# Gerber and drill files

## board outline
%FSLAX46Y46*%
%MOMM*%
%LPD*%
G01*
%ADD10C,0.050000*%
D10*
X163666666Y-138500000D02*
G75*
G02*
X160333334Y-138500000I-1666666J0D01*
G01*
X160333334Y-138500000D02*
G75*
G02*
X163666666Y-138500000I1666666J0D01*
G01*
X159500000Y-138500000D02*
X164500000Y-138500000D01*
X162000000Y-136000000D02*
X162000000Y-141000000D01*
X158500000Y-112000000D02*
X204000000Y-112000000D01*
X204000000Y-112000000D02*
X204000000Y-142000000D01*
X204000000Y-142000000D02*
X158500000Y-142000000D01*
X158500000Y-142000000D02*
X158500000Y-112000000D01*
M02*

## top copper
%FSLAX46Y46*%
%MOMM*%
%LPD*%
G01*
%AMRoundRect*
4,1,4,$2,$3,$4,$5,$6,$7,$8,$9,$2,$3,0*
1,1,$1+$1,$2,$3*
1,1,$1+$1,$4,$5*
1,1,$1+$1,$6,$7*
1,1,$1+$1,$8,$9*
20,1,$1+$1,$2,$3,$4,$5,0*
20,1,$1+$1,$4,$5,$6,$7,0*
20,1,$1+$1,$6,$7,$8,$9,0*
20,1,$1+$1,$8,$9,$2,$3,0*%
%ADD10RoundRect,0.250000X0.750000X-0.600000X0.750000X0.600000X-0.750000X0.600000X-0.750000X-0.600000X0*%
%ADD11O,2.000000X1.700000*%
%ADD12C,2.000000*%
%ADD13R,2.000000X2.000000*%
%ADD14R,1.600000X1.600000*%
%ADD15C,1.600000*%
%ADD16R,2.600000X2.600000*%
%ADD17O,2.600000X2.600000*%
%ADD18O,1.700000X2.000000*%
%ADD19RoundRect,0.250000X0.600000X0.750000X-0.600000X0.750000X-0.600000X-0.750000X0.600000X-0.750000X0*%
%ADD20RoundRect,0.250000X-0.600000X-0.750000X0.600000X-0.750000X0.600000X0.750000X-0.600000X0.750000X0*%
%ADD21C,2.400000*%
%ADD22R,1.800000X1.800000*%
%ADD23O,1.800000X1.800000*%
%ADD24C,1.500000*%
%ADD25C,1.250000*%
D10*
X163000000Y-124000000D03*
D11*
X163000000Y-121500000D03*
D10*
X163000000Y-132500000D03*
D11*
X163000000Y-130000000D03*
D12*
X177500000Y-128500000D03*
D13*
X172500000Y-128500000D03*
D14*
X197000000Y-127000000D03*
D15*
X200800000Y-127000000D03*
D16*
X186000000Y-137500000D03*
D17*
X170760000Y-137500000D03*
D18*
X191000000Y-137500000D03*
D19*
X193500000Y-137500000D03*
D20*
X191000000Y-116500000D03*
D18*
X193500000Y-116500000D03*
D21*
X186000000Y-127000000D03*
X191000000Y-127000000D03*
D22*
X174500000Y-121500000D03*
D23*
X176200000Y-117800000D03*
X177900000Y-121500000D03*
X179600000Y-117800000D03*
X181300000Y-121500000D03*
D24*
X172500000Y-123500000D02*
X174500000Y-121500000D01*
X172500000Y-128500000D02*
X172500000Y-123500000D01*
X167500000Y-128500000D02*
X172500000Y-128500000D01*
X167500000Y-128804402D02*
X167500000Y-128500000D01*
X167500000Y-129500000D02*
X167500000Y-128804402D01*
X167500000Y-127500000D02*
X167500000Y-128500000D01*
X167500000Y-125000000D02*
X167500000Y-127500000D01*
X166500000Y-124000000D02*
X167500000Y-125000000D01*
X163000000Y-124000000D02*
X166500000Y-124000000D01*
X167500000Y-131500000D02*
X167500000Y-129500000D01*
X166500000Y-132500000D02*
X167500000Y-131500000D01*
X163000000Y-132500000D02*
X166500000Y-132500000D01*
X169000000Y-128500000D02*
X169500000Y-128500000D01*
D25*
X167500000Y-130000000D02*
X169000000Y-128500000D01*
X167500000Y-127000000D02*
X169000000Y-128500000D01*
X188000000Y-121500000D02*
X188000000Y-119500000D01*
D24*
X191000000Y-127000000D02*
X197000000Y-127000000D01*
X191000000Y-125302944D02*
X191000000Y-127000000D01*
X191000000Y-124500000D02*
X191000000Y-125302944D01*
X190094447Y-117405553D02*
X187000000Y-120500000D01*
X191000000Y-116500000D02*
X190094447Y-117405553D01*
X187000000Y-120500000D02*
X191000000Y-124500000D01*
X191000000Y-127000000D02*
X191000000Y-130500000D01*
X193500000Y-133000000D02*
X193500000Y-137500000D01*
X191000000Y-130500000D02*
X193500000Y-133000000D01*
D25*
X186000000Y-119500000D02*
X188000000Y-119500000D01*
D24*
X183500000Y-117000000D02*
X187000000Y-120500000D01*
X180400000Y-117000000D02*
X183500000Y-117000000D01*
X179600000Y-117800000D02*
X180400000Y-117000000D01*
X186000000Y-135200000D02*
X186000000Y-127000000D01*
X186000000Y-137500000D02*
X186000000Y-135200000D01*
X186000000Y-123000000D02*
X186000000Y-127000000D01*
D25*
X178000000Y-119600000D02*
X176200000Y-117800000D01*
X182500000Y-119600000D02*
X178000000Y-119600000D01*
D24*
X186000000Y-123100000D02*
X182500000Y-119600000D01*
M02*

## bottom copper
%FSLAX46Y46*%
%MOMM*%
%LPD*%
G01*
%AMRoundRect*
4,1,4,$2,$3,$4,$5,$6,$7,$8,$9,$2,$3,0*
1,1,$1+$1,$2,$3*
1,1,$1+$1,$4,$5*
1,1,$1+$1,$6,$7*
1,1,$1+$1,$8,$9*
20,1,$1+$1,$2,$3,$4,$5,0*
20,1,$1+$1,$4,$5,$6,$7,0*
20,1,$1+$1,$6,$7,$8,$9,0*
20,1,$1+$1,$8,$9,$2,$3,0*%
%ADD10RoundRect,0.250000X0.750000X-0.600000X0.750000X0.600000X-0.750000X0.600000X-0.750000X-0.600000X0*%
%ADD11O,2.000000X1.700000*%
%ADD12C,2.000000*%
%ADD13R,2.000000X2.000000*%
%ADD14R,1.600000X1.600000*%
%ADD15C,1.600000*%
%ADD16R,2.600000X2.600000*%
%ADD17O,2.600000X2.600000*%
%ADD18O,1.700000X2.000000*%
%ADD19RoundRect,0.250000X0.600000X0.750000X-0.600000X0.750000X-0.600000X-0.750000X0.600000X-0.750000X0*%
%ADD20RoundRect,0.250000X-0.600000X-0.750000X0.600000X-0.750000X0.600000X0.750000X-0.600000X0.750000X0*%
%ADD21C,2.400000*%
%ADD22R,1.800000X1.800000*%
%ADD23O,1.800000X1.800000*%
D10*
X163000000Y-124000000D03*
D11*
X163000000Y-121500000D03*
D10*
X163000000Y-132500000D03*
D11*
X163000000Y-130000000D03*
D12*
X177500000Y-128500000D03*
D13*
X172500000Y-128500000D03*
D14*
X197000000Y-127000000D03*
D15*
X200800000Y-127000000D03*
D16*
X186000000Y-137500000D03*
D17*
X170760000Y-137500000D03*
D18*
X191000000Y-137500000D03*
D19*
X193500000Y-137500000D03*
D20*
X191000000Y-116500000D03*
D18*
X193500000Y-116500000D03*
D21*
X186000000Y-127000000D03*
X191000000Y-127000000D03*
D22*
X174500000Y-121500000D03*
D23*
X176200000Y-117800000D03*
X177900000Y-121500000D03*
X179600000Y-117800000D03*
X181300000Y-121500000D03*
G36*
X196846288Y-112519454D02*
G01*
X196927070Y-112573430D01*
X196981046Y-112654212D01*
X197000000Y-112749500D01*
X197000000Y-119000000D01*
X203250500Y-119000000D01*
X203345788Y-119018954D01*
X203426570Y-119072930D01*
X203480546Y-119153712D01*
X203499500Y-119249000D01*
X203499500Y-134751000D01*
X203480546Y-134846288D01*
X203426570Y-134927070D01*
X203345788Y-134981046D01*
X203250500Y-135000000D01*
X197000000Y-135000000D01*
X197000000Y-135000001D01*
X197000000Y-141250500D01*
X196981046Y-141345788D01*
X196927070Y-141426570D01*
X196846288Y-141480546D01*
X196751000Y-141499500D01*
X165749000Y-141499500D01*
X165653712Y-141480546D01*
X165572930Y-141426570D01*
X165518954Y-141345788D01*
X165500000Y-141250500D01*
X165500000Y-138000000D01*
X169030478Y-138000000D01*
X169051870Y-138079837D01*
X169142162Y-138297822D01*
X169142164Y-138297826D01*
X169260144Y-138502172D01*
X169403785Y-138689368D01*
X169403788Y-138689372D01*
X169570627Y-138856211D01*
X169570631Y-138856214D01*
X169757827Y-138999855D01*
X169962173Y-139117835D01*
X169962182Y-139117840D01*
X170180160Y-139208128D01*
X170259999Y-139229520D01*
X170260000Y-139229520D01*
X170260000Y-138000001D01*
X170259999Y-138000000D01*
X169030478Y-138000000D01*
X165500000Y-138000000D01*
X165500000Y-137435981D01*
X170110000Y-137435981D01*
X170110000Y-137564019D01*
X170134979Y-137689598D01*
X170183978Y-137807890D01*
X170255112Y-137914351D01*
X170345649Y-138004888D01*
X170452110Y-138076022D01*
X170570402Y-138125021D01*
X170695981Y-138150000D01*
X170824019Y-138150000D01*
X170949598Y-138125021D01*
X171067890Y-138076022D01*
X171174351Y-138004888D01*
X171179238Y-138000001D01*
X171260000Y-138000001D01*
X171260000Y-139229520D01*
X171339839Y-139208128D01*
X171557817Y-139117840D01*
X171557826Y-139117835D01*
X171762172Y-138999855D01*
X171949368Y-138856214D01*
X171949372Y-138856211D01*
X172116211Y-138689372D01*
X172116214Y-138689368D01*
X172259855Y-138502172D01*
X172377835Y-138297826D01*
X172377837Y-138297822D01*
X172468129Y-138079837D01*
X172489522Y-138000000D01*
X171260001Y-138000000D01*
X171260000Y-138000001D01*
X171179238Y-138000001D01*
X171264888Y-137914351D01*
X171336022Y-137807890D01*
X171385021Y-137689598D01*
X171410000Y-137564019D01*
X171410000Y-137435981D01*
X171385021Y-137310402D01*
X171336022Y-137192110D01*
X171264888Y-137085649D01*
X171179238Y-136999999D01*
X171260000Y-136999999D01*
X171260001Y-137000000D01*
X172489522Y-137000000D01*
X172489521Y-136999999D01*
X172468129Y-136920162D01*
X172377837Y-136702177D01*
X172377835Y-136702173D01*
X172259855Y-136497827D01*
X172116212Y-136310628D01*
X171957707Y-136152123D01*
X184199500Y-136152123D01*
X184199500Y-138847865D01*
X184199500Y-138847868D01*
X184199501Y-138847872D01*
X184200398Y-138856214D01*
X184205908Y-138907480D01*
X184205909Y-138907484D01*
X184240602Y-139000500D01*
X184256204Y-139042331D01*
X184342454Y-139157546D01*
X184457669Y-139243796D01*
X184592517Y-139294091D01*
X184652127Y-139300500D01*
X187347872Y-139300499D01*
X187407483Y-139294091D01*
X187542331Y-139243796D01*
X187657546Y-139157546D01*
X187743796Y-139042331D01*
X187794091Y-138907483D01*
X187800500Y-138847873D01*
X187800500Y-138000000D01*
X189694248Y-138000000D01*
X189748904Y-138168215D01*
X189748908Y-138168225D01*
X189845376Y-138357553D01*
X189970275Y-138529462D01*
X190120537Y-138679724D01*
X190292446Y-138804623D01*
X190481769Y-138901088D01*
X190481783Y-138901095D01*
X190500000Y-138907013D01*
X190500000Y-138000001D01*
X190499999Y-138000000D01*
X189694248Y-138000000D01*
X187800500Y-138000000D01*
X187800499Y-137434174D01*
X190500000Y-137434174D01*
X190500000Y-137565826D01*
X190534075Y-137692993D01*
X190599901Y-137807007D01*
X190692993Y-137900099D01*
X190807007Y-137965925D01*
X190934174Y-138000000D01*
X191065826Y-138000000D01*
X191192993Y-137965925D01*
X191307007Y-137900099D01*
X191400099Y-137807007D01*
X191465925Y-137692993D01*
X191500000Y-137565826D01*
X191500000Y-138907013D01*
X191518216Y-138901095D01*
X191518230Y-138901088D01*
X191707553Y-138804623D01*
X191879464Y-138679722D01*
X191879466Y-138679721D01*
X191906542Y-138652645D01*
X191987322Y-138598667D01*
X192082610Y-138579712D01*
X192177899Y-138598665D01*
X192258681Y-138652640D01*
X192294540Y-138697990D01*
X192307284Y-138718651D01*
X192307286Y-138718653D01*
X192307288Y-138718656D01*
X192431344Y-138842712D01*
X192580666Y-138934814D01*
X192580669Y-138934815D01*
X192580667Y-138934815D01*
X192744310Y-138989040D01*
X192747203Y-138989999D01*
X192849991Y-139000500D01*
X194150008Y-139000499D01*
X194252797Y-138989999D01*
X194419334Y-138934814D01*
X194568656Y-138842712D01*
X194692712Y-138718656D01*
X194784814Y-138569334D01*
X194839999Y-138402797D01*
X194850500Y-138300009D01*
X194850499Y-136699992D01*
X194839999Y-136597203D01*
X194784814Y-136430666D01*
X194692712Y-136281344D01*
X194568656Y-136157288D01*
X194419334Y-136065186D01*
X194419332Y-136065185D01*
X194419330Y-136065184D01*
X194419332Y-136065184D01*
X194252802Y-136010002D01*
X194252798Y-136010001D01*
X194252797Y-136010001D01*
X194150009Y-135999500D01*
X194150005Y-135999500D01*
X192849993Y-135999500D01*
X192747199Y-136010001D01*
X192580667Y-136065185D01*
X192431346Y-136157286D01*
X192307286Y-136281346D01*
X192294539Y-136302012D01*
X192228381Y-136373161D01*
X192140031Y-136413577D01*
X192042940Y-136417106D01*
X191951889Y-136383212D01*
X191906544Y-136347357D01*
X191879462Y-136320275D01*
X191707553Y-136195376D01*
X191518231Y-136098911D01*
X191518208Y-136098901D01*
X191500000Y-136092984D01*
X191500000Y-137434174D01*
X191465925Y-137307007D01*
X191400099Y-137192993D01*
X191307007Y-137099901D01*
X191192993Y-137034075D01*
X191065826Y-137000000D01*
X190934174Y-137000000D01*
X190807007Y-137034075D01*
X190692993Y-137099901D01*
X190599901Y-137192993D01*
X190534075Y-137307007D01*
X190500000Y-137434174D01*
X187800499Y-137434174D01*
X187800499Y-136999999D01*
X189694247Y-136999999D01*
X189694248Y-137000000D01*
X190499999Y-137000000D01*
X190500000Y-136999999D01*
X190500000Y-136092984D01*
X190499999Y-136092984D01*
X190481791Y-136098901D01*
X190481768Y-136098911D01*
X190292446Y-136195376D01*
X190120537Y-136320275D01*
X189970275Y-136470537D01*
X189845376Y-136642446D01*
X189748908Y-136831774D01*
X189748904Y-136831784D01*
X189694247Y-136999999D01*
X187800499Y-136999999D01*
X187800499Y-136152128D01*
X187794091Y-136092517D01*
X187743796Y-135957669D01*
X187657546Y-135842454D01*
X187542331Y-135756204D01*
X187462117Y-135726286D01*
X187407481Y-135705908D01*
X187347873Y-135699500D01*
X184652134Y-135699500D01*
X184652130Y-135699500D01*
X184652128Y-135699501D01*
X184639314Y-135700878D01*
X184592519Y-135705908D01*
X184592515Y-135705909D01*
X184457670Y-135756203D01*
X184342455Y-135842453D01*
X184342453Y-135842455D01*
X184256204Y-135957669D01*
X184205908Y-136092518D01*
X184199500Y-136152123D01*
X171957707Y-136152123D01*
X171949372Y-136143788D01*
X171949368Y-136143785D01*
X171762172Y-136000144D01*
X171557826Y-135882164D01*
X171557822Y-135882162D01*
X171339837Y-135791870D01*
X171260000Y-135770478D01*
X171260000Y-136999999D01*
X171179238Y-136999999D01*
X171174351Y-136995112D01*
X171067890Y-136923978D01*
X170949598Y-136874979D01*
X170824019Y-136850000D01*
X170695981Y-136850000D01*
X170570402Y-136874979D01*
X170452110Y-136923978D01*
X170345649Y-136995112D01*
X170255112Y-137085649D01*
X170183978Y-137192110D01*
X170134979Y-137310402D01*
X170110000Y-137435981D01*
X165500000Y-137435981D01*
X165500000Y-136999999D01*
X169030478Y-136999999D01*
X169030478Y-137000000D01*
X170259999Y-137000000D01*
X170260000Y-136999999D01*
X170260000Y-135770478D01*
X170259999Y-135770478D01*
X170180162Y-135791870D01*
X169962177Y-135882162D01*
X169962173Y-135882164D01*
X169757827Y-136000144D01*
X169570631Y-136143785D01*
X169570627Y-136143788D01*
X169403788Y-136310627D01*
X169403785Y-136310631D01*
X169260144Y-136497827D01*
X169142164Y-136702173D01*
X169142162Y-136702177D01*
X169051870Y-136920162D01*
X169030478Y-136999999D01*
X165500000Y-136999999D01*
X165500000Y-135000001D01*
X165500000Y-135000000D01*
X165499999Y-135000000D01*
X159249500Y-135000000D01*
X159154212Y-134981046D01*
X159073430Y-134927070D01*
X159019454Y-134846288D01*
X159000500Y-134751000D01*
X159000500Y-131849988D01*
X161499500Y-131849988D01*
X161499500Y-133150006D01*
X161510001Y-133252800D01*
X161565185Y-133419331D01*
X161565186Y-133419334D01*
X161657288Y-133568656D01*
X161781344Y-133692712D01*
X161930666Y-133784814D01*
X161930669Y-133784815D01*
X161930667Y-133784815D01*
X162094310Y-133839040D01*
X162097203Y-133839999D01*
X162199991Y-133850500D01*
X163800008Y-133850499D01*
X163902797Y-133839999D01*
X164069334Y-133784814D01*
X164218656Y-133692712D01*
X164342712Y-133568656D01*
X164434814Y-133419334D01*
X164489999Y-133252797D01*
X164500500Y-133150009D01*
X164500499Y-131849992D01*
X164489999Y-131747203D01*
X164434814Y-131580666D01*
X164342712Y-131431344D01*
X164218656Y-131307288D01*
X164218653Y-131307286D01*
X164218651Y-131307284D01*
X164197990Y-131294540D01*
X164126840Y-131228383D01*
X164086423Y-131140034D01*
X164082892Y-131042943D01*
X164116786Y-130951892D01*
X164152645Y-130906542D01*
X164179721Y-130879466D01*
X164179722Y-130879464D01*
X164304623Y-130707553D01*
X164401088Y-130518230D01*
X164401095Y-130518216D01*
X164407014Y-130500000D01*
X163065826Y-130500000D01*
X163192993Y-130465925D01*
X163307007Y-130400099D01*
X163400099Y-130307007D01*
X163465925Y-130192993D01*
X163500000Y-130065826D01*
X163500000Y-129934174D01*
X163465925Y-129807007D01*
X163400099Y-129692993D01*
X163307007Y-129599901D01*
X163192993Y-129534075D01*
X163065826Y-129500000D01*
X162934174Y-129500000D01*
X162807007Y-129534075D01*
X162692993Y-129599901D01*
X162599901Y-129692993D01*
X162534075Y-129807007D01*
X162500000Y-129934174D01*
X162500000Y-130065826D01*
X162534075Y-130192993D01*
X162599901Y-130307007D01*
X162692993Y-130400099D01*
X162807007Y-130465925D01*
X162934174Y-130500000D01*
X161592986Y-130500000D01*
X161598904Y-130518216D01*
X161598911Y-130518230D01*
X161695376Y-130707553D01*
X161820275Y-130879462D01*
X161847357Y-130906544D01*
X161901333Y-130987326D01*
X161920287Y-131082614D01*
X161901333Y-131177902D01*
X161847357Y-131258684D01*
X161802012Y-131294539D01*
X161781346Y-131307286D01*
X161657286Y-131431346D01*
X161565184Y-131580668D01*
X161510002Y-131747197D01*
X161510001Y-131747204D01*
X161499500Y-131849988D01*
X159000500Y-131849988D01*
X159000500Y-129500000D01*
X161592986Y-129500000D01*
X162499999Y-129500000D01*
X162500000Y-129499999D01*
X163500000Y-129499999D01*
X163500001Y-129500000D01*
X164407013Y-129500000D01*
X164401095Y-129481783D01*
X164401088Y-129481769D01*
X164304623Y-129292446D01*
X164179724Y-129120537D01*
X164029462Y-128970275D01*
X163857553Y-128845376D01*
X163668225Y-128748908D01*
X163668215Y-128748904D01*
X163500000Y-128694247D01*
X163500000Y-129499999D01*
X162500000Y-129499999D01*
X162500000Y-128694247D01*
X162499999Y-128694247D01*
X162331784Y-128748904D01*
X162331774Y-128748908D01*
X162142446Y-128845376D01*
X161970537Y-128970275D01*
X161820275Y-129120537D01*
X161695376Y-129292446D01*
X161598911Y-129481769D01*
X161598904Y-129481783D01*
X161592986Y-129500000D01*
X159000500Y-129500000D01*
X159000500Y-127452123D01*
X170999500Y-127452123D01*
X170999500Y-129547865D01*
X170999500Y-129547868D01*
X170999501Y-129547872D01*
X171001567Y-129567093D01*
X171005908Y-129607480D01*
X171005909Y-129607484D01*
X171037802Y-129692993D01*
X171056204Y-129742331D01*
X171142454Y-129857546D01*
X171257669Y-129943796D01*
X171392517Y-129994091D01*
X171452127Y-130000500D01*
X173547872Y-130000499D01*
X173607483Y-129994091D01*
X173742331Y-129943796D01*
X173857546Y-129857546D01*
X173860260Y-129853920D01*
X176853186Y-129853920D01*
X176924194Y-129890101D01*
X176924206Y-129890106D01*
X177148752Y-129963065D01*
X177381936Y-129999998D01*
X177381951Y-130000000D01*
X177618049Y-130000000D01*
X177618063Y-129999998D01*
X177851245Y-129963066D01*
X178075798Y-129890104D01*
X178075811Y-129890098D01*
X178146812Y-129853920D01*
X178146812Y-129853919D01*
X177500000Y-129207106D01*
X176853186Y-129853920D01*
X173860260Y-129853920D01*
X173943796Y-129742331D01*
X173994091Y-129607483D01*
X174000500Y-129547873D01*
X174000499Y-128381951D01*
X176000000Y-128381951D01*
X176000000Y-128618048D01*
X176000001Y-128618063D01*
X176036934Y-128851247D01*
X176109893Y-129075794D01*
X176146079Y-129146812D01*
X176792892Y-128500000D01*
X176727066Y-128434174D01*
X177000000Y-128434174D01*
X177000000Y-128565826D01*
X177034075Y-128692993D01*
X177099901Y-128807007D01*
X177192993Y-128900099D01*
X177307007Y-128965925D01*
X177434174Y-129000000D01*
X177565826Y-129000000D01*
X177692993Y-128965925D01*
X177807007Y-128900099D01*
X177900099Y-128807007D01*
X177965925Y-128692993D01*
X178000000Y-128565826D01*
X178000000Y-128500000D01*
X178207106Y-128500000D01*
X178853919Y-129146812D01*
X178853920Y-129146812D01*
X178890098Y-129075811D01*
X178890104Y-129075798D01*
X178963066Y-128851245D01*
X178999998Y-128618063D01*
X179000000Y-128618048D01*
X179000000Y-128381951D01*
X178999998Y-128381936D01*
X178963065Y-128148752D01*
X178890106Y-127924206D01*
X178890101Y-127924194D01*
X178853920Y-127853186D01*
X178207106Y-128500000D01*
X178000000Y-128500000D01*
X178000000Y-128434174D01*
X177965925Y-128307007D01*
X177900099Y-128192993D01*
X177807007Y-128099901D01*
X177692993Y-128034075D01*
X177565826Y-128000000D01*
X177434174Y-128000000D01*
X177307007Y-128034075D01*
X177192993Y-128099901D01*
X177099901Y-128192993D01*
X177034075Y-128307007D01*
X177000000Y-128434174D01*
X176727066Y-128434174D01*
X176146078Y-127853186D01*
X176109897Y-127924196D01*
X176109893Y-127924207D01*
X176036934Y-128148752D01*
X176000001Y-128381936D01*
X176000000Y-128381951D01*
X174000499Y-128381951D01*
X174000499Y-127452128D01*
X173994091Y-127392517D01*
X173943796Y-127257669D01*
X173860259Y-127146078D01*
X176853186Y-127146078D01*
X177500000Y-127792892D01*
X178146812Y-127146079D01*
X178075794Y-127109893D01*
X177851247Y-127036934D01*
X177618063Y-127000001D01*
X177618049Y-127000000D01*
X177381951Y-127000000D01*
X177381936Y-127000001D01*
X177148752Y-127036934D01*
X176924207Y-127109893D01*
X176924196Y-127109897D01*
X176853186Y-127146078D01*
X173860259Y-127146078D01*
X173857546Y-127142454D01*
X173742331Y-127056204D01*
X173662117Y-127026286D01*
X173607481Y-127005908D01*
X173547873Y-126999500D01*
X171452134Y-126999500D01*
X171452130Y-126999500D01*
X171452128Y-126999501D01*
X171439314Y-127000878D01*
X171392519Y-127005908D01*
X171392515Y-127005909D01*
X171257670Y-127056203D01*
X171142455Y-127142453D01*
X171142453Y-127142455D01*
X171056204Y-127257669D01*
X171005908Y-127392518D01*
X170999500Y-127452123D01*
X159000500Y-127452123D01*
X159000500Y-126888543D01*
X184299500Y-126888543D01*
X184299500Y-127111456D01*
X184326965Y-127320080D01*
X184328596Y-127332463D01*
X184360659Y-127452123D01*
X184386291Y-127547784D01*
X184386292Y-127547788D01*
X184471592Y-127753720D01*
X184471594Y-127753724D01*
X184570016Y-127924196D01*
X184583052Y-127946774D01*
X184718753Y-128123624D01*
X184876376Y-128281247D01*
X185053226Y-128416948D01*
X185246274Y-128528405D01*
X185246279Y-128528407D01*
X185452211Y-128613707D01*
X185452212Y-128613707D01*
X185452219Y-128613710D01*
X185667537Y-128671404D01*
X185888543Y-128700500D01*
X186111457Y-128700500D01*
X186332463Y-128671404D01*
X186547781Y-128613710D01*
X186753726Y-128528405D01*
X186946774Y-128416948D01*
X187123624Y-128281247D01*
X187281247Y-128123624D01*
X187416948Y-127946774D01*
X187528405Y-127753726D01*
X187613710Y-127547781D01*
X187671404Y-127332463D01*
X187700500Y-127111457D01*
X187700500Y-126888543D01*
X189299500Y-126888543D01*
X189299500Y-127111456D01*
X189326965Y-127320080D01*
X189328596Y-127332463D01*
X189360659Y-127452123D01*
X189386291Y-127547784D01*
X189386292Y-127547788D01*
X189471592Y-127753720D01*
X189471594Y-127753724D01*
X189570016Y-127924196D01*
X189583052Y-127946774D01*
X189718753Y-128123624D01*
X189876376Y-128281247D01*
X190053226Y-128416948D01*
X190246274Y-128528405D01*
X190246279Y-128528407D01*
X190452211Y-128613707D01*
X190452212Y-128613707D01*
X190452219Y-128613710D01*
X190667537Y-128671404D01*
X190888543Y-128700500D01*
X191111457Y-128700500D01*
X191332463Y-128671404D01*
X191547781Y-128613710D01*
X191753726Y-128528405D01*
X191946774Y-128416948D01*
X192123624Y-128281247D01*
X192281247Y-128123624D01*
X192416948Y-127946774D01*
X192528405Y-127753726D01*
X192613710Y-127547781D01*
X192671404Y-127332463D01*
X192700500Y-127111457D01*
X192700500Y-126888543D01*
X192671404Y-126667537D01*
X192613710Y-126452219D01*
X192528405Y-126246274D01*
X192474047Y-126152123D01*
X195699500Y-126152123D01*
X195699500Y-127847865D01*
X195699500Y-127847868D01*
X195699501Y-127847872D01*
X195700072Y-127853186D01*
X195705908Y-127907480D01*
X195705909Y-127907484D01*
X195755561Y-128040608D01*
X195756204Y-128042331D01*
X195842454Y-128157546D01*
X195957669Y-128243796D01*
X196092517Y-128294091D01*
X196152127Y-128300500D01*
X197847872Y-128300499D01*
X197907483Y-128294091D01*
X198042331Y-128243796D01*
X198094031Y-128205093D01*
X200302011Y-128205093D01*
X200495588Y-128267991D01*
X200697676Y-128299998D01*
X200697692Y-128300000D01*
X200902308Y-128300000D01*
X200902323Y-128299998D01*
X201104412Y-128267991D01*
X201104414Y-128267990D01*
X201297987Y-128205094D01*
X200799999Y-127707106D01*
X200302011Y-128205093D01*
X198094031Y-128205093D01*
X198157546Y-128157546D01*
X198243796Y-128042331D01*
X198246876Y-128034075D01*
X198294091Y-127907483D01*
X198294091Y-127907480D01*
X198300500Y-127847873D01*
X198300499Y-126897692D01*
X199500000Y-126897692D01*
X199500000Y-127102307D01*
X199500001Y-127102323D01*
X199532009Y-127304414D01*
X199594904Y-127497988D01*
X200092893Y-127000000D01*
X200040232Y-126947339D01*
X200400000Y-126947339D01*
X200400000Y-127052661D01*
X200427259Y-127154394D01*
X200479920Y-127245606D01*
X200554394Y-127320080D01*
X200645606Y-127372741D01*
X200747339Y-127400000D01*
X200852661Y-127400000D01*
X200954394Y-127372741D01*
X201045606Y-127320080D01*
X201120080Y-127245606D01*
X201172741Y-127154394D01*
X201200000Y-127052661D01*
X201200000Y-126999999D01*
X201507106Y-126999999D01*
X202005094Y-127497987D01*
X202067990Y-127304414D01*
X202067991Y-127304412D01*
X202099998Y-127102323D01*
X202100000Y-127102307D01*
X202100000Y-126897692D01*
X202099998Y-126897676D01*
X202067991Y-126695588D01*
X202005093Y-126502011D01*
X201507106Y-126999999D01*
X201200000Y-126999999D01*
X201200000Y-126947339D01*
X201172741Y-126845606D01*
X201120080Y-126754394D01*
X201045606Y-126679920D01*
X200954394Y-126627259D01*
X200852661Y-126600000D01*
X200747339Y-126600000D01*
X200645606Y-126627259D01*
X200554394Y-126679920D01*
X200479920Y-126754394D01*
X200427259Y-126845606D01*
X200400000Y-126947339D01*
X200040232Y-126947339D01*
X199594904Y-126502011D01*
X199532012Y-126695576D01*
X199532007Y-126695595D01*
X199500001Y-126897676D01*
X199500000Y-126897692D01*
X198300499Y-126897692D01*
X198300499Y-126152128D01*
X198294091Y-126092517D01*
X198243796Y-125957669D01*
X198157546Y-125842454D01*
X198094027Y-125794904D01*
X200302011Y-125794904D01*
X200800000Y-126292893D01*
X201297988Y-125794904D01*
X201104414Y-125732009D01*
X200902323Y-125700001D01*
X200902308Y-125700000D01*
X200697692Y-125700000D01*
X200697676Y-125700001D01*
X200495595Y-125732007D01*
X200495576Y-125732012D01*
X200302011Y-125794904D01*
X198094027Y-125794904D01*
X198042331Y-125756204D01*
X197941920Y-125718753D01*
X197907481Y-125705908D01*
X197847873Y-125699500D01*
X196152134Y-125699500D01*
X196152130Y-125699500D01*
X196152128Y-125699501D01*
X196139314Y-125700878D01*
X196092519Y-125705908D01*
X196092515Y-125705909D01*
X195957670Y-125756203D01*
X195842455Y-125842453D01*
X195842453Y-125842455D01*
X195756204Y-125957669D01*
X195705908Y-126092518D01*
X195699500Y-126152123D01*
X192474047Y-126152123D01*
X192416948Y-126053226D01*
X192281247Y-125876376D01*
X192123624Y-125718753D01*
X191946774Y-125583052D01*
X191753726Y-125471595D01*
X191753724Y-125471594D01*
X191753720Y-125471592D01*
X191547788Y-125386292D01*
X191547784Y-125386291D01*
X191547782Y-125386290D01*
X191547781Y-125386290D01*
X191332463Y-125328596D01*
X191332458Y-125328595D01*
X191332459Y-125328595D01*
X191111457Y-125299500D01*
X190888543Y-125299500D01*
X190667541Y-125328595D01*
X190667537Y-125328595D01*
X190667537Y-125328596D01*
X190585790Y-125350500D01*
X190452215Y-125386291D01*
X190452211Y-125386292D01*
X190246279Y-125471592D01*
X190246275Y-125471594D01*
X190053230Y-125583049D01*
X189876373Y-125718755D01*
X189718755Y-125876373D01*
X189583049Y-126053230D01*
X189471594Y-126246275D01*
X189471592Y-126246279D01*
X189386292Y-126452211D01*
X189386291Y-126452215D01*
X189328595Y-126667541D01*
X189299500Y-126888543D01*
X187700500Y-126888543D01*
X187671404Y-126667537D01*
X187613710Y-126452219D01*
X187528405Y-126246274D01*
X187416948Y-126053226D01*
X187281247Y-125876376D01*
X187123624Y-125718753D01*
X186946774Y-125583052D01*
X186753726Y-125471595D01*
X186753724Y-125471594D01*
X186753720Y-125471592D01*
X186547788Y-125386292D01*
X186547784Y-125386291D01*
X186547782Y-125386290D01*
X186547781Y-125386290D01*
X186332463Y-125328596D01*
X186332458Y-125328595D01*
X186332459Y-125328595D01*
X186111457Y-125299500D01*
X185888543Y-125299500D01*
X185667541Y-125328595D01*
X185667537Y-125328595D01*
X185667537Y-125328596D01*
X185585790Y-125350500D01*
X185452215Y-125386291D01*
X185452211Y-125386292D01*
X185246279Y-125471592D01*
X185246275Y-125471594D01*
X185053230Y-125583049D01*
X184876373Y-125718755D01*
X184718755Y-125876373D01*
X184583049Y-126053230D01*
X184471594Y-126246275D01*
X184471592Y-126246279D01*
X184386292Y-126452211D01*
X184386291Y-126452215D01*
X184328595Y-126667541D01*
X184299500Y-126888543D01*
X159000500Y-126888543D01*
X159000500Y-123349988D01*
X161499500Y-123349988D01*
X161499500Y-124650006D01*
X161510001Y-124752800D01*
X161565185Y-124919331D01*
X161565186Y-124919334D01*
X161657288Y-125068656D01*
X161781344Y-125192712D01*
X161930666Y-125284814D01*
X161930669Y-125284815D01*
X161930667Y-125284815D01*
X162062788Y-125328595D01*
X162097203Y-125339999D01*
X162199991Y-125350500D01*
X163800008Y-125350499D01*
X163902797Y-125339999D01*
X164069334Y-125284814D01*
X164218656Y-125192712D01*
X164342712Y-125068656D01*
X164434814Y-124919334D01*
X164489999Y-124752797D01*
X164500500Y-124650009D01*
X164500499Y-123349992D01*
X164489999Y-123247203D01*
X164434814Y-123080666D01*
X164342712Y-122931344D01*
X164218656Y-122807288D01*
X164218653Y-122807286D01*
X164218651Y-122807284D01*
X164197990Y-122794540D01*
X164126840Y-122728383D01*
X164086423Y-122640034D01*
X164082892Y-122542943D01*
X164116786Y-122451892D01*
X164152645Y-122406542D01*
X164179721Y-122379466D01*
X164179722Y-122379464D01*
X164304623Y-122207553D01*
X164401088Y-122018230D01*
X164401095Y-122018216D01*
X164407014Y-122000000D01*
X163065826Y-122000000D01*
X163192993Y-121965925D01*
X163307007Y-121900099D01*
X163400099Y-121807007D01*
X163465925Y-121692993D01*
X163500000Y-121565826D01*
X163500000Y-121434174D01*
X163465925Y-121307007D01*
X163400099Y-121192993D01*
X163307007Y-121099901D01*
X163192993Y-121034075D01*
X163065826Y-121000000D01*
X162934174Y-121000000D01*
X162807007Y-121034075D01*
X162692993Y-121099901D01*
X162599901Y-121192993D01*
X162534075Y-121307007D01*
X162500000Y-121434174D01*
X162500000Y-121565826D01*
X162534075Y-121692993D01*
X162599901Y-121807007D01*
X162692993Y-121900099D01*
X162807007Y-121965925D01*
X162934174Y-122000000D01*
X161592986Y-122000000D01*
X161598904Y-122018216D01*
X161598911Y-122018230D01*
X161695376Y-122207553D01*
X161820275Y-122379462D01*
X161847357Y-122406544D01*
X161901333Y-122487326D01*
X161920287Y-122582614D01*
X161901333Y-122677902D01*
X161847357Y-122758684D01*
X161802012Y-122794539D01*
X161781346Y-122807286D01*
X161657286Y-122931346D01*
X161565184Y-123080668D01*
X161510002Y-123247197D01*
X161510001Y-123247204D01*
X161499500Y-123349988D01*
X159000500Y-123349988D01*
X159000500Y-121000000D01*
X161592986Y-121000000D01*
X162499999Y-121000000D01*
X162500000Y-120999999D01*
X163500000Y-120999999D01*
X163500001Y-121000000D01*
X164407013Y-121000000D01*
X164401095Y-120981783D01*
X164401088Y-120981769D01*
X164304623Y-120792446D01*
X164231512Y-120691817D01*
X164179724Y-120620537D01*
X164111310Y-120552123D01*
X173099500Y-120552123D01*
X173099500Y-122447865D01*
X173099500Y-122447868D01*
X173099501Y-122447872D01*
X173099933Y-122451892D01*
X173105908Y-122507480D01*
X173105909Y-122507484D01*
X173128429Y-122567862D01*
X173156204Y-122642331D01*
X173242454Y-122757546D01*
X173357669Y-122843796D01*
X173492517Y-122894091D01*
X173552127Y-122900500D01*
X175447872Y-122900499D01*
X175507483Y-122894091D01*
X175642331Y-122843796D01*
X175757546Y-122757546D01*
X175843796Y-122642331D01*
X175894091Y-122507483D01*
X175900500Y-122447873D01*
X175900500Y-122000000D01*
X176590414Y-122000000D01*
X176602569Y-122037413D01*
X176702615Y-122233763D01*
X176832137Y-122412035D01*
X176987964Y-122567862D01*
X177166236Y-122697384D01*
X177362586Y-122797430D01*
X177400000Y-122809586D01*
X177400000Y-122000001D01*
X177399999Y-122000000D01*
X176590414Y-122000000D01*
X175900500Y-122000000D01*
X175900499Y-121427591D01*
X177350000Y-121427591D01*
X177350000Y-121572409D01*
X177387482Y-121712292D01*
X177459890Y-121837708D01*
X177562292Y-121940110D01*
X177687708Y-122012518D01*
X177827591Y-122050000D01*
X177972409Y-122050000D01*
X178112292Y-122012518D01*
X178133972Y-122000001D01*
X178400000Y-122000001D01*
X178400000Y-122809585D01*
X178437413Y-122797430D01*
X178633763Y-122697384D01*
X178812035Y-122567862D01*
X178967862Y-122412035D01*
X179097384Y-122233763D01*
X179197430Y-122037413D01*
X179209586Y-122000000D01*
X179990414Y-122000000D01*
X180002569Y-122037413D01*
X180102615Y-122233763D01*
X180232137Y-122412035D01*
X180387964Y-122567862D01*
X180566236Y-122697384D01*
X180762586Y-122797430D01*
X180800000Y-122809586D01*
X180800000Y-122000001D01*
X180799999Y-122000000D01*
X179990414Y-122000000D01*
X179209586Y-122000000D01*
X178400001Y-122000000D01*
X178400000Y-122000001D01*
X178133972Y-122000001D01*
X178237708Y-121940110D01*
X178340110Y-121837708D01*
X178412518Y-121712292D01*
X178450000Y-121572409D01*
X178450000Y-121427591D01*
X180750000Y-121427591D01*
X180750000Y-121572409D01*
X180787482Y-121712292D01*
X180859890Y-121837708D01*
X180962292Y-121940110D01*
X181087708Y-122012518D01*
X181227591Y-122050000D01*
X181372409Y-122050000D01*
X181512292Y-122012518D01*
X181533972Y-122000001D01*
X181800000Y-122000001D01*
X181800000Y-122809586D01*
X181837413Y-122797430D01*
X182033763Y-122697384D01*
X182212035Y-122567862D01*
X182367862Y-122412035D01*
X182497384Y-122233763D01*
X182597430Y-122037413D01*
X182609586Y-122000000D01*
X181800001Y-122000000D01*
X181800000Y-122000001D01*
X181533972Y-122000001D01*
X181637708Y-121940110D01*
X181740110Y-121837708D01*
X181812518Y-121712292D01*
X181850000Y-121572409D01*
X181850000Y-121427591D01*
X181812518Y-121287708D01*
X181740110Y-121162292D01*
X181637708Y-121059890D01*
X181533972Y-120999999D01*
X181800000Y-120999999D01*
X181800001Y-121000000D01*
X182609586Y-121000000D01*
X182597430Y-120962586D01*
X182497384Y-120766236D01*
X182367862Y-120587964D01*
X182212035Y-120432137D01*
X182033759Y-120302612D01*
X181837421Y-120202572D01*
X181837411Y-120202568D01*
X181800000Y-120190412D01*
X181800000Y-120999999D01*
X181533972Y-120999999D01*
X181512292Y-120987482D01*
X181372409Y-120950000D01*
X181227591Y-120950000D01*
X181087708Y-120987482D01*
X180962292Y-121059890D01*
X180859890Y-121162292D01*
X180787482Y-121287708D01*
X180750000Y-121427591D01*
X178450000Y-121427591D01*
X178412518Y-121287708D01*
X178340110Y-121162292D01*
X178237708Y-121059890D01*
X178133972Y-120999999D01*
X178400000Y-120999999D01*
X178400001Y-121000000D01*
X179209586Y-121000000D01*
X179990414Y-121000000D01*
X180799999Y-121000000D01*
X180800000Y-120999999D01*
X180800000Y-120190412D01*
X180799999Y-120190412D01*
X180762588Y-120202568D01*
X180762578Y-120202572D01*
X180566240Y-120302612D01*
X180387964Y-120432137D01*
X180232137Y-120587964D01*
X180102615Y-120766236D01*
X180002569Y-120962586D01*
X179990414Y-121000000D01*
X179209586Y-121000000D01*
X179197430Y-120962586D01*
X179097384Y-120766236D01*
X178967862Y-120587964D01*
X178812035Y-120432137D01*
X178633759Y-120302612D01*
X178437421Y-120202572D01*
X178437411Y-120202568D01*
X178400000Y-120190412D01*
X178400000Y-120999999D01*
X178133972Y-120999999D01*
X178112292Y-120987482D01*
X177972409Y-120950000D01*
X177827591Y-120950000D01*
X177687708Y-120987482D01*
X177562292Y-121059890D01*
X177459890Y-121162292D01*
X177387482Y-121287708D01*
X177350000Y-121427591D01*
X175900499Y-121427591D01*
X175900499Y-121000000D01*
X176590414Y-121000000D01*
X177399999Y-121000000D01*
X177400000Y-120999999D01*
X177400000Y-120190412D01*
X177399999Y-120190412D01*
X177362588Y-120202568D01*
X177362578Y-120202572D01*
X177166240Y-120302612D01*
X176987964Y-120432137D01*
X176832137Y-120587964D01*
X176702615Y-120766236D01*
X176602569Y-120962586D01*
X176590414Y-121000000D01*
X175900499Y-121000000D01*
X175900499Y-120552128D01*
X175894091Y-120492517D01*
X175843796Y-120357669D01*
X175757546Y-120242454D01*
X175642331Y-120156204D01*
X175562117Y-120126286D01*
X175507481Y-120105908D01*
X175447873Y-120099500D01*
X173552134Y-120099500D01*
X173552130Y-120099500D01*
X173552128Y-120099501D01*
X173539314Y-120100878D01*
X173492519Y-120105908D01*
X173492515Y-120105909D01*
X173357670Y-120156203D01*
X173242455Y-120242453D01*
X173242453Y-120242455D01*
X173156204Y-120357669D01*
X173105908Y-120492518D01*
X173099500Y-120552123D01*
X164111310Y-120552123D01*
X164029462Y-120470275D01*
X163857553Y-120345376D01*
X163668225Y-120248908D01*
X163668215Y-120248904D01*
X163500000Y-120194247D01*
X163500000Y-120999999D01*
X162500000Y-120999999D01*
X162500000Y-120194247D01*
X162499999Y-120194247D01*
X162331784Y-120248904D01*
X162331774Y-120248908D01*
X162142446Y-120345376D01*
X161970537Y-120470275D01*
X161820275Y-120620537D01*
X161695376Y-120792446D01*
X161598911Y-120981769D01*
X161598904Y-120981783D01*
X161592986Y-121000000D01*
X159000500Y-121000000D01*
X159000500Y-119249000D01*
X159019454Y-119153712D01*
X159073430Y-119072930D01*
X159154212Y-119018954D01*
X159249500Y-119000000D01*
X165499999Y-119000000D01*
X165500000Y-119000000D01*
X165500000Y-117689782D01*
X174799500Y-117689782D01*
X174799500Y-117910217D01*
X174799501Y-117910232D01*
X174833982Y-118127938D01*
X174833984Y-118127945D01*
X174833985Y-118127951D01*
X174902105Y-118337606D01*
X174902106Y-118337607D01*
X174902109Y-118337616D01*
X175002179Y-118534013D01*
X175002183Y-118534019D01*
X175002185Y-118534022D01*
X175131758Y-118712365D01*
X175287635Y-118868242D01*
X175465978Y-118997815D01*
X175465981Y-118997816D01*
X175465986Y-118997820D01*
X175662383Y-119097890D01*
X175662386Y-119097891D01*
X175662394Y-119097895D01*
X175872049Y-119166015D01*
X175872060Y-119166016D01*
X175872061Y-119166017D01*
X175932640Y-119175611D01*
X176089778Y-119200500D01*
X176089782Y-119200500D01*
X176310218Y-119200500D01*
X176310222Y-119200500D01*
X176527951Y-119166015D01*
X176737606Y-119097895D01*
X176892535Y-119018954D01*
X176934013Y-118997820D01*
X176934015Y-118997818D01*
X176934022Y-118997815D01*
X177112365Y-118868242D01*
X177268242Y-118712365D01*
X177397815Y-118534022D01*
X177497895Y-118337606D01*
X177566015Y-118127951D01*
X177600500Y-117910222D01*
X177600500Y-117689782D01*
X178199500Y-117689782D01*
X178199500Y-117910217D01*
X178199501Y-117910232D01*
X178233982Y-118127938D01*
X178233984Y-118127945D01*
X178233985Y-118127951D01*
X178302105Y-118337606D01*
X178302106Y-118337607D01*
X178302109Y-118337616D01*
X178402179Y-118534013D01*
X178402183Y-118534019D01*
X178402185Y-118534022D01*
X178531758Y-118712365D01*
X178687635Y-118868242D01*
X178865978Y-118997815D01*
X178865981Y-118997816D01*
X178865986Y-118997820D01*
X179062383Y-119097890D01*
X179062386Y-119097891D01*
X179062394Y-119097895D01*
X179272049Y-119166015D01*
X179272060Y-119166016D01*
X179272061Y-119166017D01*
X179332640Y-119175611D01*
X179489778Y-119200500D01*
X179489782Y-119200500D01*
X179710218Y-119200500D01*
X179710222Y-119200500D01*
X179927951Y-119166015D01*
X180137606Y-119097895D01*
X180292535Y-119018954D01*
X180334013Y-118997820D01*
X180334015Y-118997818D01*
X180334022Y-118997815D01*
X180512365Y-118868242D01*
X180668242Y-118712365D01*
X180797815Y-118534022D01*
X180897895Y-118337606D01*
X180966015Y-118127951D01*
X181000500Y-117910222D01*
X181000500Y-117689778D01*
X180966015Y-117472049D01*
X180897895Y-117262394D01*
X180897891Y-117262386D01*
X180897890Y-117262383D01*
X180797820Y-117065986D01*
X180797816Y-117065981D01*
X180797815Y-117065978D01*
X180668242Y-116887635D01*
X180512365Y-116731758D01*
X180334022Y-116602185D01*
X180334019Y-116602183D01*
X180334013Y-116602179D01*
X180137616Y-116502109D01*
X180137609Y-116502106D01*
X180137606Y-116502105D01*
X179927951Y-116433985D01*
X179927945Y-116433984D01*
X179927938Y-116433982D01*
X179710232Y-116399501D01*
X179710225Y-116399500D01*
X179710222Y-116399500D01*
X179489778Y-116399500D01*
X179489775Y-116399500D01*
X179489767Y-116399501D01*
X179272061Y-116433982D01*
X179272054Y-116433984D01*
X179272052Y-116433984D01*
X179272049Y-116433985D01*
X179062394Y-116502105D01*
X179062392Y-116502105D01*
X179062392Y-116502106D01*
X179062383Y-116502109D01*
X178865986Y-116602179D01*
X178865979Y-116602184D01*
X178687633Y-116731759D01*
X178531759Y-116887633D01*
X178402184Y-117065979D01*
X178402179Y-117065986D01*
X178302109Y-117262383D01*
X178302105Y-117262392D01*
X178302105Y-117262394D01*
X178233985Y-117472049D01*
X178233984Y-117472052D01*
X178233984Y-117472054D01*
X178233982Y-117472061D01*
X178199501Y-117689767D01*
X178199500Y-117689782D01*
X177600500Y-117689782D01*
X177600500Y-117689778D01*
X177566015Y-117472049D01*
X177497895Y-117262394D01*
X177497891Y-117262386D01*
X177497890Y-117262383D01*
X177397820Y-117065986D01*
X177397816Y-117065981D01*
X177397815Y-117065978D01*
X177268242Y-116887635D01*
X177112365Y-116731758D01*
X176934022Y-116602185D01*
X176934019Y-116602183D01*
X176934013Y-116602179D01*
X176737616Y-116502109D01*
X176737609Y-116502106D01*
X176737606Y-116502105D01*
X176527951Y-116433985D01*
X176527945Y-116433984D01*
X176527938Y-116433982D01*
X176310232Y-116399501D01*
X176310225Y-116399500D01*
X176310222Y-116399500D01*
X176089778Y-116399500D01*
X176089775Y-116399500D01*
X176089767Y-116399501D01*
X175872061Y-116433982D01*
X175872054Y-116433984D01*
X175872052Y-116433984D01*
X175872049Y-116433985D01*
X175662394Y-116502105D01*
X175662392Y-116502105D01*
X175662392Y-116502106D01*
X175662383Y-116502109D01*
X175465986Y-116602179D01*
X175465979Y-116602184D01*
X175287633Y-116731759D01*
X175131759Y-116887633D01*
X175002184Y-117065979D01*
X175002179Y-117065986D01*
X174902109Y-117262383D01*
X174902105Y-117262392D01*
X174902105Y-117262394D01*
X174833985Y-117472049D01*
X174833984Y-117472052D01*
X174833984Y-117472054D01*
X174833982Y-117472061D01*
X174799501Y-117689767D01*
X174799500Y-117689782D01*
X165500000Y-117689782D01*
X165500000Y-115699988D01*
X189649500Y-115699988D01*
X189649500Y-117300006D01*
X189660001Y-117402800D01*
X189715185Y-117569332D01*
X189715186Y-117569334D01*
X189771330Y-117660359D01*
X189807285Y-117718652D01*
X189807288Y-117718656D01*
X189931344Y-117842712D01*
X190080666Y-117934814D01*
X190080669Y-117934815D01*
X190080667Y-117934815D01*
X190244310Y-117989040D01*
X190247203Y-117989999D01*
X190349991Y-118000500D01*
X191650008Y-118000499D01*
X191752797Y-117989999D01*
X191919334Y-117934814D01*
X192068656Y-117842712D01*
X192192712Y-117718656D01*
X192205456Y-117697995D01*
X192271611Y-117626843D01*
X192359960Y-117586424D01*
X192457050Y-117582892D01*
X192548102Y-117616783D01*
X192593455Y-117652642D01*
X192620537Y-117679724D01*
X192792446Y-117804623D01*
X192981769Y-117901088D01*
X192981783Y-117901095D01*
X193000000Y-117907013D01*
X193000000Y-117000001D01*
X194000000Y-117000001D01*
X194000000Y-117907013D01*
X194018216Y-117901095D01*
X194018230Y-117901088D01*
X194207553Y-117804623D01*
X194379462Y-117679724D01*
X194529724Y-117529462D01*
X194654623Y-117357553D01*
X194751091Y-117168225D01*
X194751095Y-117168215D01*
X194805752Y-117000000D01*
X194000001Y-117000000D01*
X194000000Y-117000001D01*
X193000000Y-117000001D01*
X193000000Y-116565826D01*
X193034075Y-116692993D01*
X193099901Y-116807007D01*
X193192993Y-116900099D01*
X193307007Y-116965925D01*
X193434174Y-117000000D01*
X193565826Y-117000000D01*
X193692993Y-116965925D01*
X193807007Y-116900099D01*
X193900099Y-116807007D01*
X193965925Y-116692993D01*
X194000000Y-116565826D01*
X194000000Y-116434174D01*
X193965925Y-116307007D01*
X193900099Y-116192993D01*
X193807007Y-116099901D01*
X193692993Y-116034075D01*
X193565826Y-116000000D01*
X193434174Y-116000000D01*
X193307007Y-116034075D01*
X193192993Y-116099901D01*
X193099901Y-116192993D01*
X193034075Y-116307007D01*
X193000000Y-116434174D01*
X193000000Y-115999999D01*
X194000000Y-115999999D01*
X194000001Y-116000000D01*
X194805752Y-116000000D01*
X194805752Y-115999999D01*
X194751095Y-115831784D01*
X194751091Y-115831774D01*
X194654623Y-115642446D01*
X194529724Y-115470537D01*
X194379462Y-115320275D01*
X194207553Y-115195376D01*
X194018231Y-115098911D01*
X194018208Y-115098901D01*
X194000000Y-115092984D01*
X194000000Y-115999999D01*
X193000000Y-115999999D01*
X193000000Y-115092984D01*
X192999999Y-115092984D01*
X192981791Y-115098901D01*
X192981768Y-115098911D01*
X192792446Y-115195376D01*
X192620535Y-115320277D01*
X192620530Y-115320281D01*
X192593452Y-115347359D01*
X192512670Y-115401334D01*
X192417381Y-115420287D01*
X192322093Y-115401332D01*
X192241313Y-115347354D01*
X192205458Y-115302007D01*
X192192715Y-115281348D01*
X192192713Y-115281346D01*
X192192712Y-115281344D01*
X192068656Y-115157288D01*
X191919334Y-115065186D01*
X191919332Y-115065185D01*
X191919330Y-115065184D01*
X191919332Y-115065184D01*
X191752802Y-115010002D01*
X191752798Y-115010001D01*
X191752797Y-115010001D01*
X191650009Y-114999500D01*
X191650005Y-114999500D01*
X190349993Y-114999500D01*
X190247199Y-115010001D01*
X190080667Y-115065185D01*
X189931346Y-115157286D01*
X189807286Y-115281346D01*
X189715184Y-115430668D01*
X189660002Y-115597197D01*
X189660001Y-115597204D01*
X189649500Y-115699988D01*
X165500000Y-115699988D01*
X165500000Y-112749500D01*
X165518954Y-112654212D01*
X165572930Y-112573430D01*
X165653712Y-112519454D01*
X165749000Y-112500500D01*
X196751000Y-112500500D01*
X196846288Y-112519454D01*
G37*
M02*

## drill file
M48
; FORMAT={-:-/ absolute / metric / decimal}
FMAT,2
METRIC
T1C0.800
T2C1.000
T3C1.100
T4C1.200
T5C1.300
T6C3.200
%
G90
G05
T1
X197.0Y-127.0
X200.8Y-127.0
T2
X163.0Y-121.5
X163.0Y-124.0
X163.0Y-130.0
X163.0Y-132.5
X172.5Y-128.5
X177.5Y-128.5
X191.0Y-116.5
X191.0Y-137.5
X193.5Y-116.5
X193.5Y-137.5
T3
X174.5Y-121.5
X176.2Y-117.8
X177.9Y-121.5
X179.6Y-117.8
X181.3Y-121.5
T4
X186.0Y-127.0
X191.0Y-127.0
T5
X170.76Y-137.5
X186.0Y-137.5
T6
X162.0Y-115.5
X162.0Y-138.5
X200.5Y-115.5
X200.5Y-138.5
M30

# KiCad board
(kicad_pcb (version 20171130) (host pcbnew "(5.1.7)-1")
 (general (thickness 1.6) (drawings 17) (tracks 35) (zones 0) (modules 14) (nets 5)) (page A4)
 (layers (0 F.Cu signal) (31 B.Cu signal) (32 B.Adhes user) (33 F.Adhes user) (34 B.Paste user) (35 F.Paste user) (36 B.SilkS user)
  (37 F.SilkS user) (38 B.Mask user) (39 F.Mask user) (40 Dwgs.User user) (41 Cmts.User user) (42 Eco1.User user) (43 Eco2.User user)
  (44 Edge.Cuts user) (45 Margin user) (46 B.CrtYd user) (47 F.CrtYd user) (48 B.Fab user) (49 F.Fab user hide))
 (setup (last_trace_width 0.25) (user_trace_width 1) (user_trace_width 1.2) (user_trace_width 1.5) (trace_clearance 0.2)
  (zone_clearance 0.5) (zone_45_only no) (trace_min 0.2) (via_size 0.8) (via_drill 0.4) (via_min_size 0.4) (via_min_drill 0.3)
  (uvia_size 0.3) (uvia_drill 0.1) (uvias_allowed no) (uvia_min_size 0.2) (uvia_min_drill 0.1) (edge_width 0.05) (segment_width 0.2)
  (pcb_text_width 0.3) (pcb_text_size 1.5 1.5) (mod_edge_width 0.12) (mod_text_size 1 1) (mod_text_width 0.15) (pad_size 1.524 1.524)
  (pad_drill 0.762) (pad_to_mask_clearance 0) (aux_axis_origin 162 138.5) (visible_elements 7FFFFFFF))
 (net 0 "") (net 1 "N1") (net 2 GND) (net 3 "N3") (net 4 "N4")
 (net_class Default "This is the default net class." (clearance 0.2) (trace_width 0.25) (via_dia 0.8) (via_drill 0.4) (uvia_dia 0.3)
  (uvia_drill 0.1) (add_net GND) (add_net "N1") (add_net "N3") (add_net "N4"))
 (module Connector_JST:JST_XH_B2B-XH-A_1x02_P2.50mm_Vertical (layer F.Cu) (at 163 124 90)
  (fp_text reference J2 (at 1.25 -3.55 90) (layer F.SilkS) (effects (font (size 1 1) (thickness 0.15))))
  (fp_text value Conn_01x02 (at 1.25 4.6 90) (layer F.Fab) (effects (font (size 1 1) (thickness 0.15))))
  (pad 1 thru_hole roundrect (at 0 0 90) (size 1.7 2) (drill 1) (layers *.Cu *.Mask) (roundrect_rratio 0.1470588235294118) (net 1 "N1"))
  (pad 2 thru_hole oval (at 2.5 0 90) (size 1.7 2) (drill 1) (layers *.Cu *.Mask) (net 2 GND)))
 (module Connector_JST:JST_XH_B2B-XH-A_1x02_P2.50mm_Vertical (layer F.Cu) (at 163 132.5 90)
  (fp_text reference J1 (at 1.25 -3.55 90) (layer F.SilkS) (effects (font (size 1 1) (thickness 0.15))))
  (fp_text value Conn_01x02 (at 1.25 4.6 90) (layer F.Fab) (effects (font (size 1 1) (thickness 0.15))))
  (pad 1 thru_hole roundrect (at 0 0 90) (size 1.7 2) (drill 1) (layers *.Cu *.Mask) (roundrect_rratio 0.1470588235294118) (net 1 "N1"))
  (pad 2 thru_hole oval (at 2.5 0 90) (size 1.7 2) (drill 1) (layers *.Cu *.Mask) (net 2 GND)))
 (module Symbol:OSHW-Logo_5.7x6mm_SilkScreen (layer F.Cu) (at 168.5 116.5)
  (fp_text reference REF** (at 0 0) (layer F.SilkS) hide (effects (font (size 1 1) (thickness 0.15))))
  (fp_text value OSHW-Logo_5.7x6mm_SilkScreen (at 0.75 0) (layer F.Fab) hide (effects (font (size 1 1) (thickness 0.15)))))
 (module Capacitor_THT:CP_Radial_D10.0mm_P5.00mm (layer F.Cu) (at 172.5 128.5)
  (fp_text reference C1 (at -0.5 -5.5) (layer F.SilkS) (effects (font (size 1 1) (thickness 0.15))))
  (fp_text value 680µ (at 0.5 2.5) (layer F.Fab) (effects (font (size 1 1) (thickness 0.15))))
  (pad 2 thru_hole circle (at 5 0) (size 2 2) (drill 1) (layers *.Cu *.Mask) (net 2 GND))
  (pad 1 thru_hole rect (at 0 0) (size 2 2) (drill 1) (layers *.Cu *.Mask) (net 1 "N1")))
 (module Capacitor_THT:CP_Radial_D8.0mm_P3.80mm (layer F.Cu) (at 197 127)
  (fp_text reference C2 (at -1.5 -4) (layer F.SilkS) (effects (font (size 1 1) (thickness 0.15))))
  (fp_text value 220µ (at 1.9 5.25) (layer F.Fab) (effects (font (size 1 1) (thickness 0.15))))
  (pad 1 thru_hole rect (at 0 0) (size 1.6 1.6) (drill 0.8) (layers *.Cu *.Mask) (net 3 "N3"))
  (pad 2 thru_hole circle (at 3.8 0) (size 1.6 1.6) (drill 0.8) (layers *.Cu *.Mask) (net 2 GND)))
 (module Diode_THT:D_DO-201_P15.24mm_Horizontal (layer F.Cu) (at 186 137.5 180)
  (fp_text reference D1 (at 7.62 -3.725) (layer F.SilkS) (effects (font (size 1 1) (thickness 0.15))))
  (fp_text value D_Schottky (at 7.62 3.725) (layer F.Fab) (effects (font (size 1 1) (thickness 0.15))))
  (pad 1 thru_hole rect (at 0 0 180) (size 2.6 2.6) (drill 1.3) (layers *.Cu *.Mask) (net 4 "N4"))
  (pad 2 thru_hole oval (at 15.24 0 180) (size 2.6 2.6) (drill 1.3) (layers *.Cu *.Mask) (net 2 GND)))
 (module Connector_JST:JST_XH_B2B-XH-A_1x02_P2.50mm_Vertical (layer F.Cu) (at 193.5 137.5 180)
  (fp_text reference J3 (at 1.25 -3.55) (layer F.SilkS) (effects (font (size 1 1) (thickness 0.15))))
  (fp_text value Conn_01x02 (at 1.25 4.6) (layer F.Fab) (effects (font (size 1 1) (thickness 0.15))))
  (pad 2 thru_hole oval (at 2.5 0 180) (size 1.7 2) (drill 1) (layers *.Cu *.Mask) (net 2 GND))
  (pad 1 thru_hole roundrect (at 0 0 180) (size 1.7 2) (drill 1) (layers *.Cu *.Mask) (roundrect_rratio 0.1470588235294118) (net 3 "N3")))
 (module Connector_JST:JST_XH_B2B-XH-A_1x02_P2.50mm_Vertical (layer F.Cu) (at 191 116.5)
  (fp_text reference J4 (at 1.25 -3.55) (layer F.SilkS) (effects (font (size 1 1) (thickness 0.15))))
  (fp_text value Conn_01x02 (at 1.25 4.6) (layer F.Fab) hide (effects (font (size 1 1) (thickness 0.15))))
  (pad 1 thru_hole roundrect (at 0 0) (size 1.7 2) (drill 1) (layers *.Cu *.Mask) (roundrect_rratio 0.1470588235294118) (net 3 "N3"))
  (pad 2 thru_hole oval (at 2.5 0) (size 1.7 2) (drill 1) (layers *.Cu *.Mask) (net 2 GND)))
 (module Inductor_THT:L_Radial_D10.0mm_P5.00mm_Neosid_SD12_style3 (layer F.Cu) (at 186 127)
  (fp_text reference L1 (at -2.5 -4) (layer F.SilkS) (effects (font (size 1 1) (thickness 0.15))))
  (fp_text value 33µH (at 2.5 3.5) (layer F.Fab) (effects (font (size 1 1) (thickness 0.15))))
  (pad 1 thru_hole circle (at 0 0) (size 2.4 2.4) (drill 1.2) (layers *.Cu *.Mask) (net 4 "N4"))
  (pad 2 thru_hole circle (at 5 0) (size 2.4 2.4) (drill 1.2) (layers *.Cu *.Mask) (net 3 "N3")))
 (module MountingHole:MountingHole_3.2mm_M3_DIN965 (layer F.Cu) (at 200.5 115.5)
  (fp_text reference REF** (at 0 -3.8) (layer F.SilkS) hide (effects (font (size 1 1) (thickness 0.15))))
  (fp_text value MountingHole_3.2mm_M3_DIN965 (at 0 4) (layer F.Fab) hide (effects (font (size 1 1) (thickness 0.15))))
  (pad 1 np_thru_hole circle (at 0 0) (size 3.2 3.2) (drill 3.2) (layers *.Cu *.Mask)))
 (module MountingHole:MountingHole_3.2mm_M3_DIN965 (layer F.Cu) (at 200.5 138.5)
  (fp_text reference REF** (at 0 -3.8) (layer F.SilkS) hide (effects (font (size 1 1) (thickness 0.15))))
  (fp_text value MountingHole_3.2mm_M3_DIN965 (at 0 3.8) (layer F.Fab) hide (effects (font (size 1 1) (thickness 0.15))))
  (pad 1 np_thru_hole circle (at 0 0) (size 3.2 3.2) (drill 3.2) (layers *.Cu *.Mask)))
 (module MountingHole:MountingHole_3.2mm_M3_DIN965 (layer F.Cu) (at 162 138.5)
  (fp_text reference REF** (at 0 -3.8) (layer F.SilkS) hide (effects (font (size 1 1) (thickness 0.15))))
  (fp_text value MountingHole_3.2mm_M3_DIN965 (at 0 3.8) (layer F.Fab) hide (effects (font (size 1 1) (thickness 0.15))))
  (pad 1 np_thru_hole circle (at 0 0) (size 3.2 3.2) (drill 3.2) (layers *.Cu *.Mask)))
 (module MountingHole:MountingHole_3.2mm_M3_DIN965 (layer F.Cu) (at 162 115.5)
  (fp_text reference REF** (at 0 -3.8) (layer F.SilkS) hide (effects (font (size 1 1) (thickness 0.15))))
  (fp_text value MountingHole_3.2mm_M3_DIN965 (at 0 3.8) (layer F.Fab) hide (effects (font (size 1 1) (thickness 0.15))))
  (pad 1 np_thru_hole circle (at 0 0) (size 3.2 3.2) (drill 3.2) (layers *.Cu *.Mask)))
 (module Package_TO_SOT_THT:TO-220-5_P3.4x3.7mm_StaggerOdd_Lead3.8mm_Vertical (layer F.Cu) (at 174.5 121.5)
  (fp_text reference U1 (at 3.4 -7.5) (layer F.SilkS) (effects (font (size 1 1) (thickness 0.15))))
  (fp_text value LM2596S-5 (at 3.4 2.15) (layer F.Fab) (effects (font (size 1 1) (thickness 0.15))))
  (pad 1 thru_hole rect (at 0 0) (size 1.8 1.8) (drill 1.1) (layers *.Cu *.Mask) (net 1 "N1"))
  (pad 2 thru_hole oval (at 1.7 -3.7) (size 1.8 1.8) (drill 1.1) (layers *.Cu *.Mask) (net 4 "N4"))
  (pad 3 thru_hole oval (at 3.4 0) (size 1.8 1.8) (drill 1.1) (layers *.Cu *.Mask) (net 2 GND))
  (pad 4 thru_hole oval (at 5.1 -3.7) (size 1.8 1.8) (drill 1.1) (layers *.Cu *.Mask) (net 3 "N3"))
  (pad 5 thru_hole oval (at 6.8 0) (size 1.8 1.8) (drill 1.1) (layers *.Cu *.Mask) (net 2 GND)))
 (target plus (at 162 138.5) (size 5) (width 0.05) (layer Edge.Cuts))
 (gr_line (start 158.5 112) (end 204 112) (layer Edge.Cuts) (width 0.05))
 (gr_line (start 204 112) (end 204 142) (layer Edge.Cuts) (width 0.05))
 (gr_line (start 204 142) (end 158.5 142) (layer Edge.Cuts) (width 0.05))
 (gr_line (start 158.5 142) (end 158.5 112) (layer Edge.Cuts) (width 0.05))
 (segment (start 172.5 123.5) (end 174.5 121.5) (width 1.5) (layer F.Cu) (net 1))
 (segment (start 172.5 128.5) (end 172.5 123.5) (width 1.5) (layer F.Cu) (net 1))
 (segment (start 167.5 128.5) (end 172.5 128.5) (width 1.5) (layer F.Cu) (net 1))
 (segment (start 167.5 128.804402) (end 167.5 128.5) (width 1.5) (layer F.Cu) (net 1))
 (segment (start 167.5 129.5) (end 167.5 128.804402) (width 1.5) (layer F.Cu) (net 1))
 (segment (start 167.5 127.5) (end 167.5 128.5) (width 1.5) (layer F.Cu) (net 1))
 (segment (start 167.5 125) (end 167.5 127.5) (width 1.5) (layer F.Cu) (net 1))
 (segment (start 166.5 124) (end 167.5 125) (width 1.5) (layer F.Cu) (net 1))
 (segment (start 163 124) (end 166.5 124) (width 1.5) (layer F.Cu) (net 1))
 (segment (start 167.5 131.5) (end 167.5 129.5) (width 1.5) (layer F.Cu) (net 1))
 (segment (start 166.5 132.5) (end 167.5 131.5) (width 1.5) (layer F.Cu) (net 1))
 (segment (start 163 132.5) (end 166.5 132.5) (width 1.5) (layer F.Cu) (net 1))
 (segment (start 169 128.5) (end 169.5 128.5) (width 1.5) (layer F.Cu) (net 1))
 (segment (start 167.5 130) (end 169 128.5) (width 1.25) (layer F.Cu) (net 1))
 (segment (start 167.5 127) (end 169 128.5) (width 1.25) (layer F.Cu) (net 1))
 (segment (start 188 121.5) (end 188 119.5) (width 1.25) (layer F.Cu) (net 3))
 (segment (start 191 127) (end 197 127) (width 1.5) (layer F.Cu) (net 3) (status 30))
 (segment (start 191 125.302944) (end 191 127) (width 1.5) (layer F.Cu) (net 3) (status 20))
 (segment (start 191 124.5) (end 191 125.302944) (width 1.5) (layer F.Cu) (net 3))
 (segment (start 190.094447 117.405553) (end 187 120.5) (width 1.5) (layer F.Cu) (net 3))
 (segment (start 191 116.5) (end 190.094447 117.405553) (width 1.5) (layer F.Cu) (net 3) (status 10))
 (segment (start 187 120.5) (end 191 124.5) (width 1.5) (layer F.Cu) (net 3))
 (segment (start 191 127) (end 191 130.5) (width 1.5) (layer F.Cu) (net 3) (status 10))
 (segment (start 193.5 133) (end 193.5 137.5) (width 1.5) (layer F.Cu) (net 3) (status 20))
 (segment (start 191 130.5) (end 193.5 133) (width 1.5) (layer F.Cu) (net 3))
 (segment (start 186 119.5) (end 188 119.5) (width 1.25) (layer F.Cu) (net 3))
 (segment (start 183.5 117) (end 187 120.5) (width 1.5) (layer F.Cu) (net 3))
 (segment (start 180.4 117) (end 183.5 117) (width 1.5) (layer F.Cu) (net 3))
 (segment (start 179.6 117.8) (end 180.4 117) (width 1.5) (layer F.Cu) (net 3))
 (segment (start 186 135.2) (end 186 127) (width 1.5) (layer F.Cu) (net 4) (status 20))
 (segment (start 186 137.5) (end 186 135.2) (width 1.5) (layer F.Cu) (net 4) (status 10))
 (segment (start 186 123) (end 186 127) (width 1.5) (layer F.Cu) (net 4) (status 20))
 (segment (start 178 119.6) (end 176.2 117.8) (width 1.25) (layer F.Cu) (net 4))
 (segment (start 182.5 119.6) (end 178 119.6) (width 1.25) (layer F.Cu) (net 4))
 (segment (start 186 123.1) (end 182.5 119.6) (width 1.5) (layer F.Cu) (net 4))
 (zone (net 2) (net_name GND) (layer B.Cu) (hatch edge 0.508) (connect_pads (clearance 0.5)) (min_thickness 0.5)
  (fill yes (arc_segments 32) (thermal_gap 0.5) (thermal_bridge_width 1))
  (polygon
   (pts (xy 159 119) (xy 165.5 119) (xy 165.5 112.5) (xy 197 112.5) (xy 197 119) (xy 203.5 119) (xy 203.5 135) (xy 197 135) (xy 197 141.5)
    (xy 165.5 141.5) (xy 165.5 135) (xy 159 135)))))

